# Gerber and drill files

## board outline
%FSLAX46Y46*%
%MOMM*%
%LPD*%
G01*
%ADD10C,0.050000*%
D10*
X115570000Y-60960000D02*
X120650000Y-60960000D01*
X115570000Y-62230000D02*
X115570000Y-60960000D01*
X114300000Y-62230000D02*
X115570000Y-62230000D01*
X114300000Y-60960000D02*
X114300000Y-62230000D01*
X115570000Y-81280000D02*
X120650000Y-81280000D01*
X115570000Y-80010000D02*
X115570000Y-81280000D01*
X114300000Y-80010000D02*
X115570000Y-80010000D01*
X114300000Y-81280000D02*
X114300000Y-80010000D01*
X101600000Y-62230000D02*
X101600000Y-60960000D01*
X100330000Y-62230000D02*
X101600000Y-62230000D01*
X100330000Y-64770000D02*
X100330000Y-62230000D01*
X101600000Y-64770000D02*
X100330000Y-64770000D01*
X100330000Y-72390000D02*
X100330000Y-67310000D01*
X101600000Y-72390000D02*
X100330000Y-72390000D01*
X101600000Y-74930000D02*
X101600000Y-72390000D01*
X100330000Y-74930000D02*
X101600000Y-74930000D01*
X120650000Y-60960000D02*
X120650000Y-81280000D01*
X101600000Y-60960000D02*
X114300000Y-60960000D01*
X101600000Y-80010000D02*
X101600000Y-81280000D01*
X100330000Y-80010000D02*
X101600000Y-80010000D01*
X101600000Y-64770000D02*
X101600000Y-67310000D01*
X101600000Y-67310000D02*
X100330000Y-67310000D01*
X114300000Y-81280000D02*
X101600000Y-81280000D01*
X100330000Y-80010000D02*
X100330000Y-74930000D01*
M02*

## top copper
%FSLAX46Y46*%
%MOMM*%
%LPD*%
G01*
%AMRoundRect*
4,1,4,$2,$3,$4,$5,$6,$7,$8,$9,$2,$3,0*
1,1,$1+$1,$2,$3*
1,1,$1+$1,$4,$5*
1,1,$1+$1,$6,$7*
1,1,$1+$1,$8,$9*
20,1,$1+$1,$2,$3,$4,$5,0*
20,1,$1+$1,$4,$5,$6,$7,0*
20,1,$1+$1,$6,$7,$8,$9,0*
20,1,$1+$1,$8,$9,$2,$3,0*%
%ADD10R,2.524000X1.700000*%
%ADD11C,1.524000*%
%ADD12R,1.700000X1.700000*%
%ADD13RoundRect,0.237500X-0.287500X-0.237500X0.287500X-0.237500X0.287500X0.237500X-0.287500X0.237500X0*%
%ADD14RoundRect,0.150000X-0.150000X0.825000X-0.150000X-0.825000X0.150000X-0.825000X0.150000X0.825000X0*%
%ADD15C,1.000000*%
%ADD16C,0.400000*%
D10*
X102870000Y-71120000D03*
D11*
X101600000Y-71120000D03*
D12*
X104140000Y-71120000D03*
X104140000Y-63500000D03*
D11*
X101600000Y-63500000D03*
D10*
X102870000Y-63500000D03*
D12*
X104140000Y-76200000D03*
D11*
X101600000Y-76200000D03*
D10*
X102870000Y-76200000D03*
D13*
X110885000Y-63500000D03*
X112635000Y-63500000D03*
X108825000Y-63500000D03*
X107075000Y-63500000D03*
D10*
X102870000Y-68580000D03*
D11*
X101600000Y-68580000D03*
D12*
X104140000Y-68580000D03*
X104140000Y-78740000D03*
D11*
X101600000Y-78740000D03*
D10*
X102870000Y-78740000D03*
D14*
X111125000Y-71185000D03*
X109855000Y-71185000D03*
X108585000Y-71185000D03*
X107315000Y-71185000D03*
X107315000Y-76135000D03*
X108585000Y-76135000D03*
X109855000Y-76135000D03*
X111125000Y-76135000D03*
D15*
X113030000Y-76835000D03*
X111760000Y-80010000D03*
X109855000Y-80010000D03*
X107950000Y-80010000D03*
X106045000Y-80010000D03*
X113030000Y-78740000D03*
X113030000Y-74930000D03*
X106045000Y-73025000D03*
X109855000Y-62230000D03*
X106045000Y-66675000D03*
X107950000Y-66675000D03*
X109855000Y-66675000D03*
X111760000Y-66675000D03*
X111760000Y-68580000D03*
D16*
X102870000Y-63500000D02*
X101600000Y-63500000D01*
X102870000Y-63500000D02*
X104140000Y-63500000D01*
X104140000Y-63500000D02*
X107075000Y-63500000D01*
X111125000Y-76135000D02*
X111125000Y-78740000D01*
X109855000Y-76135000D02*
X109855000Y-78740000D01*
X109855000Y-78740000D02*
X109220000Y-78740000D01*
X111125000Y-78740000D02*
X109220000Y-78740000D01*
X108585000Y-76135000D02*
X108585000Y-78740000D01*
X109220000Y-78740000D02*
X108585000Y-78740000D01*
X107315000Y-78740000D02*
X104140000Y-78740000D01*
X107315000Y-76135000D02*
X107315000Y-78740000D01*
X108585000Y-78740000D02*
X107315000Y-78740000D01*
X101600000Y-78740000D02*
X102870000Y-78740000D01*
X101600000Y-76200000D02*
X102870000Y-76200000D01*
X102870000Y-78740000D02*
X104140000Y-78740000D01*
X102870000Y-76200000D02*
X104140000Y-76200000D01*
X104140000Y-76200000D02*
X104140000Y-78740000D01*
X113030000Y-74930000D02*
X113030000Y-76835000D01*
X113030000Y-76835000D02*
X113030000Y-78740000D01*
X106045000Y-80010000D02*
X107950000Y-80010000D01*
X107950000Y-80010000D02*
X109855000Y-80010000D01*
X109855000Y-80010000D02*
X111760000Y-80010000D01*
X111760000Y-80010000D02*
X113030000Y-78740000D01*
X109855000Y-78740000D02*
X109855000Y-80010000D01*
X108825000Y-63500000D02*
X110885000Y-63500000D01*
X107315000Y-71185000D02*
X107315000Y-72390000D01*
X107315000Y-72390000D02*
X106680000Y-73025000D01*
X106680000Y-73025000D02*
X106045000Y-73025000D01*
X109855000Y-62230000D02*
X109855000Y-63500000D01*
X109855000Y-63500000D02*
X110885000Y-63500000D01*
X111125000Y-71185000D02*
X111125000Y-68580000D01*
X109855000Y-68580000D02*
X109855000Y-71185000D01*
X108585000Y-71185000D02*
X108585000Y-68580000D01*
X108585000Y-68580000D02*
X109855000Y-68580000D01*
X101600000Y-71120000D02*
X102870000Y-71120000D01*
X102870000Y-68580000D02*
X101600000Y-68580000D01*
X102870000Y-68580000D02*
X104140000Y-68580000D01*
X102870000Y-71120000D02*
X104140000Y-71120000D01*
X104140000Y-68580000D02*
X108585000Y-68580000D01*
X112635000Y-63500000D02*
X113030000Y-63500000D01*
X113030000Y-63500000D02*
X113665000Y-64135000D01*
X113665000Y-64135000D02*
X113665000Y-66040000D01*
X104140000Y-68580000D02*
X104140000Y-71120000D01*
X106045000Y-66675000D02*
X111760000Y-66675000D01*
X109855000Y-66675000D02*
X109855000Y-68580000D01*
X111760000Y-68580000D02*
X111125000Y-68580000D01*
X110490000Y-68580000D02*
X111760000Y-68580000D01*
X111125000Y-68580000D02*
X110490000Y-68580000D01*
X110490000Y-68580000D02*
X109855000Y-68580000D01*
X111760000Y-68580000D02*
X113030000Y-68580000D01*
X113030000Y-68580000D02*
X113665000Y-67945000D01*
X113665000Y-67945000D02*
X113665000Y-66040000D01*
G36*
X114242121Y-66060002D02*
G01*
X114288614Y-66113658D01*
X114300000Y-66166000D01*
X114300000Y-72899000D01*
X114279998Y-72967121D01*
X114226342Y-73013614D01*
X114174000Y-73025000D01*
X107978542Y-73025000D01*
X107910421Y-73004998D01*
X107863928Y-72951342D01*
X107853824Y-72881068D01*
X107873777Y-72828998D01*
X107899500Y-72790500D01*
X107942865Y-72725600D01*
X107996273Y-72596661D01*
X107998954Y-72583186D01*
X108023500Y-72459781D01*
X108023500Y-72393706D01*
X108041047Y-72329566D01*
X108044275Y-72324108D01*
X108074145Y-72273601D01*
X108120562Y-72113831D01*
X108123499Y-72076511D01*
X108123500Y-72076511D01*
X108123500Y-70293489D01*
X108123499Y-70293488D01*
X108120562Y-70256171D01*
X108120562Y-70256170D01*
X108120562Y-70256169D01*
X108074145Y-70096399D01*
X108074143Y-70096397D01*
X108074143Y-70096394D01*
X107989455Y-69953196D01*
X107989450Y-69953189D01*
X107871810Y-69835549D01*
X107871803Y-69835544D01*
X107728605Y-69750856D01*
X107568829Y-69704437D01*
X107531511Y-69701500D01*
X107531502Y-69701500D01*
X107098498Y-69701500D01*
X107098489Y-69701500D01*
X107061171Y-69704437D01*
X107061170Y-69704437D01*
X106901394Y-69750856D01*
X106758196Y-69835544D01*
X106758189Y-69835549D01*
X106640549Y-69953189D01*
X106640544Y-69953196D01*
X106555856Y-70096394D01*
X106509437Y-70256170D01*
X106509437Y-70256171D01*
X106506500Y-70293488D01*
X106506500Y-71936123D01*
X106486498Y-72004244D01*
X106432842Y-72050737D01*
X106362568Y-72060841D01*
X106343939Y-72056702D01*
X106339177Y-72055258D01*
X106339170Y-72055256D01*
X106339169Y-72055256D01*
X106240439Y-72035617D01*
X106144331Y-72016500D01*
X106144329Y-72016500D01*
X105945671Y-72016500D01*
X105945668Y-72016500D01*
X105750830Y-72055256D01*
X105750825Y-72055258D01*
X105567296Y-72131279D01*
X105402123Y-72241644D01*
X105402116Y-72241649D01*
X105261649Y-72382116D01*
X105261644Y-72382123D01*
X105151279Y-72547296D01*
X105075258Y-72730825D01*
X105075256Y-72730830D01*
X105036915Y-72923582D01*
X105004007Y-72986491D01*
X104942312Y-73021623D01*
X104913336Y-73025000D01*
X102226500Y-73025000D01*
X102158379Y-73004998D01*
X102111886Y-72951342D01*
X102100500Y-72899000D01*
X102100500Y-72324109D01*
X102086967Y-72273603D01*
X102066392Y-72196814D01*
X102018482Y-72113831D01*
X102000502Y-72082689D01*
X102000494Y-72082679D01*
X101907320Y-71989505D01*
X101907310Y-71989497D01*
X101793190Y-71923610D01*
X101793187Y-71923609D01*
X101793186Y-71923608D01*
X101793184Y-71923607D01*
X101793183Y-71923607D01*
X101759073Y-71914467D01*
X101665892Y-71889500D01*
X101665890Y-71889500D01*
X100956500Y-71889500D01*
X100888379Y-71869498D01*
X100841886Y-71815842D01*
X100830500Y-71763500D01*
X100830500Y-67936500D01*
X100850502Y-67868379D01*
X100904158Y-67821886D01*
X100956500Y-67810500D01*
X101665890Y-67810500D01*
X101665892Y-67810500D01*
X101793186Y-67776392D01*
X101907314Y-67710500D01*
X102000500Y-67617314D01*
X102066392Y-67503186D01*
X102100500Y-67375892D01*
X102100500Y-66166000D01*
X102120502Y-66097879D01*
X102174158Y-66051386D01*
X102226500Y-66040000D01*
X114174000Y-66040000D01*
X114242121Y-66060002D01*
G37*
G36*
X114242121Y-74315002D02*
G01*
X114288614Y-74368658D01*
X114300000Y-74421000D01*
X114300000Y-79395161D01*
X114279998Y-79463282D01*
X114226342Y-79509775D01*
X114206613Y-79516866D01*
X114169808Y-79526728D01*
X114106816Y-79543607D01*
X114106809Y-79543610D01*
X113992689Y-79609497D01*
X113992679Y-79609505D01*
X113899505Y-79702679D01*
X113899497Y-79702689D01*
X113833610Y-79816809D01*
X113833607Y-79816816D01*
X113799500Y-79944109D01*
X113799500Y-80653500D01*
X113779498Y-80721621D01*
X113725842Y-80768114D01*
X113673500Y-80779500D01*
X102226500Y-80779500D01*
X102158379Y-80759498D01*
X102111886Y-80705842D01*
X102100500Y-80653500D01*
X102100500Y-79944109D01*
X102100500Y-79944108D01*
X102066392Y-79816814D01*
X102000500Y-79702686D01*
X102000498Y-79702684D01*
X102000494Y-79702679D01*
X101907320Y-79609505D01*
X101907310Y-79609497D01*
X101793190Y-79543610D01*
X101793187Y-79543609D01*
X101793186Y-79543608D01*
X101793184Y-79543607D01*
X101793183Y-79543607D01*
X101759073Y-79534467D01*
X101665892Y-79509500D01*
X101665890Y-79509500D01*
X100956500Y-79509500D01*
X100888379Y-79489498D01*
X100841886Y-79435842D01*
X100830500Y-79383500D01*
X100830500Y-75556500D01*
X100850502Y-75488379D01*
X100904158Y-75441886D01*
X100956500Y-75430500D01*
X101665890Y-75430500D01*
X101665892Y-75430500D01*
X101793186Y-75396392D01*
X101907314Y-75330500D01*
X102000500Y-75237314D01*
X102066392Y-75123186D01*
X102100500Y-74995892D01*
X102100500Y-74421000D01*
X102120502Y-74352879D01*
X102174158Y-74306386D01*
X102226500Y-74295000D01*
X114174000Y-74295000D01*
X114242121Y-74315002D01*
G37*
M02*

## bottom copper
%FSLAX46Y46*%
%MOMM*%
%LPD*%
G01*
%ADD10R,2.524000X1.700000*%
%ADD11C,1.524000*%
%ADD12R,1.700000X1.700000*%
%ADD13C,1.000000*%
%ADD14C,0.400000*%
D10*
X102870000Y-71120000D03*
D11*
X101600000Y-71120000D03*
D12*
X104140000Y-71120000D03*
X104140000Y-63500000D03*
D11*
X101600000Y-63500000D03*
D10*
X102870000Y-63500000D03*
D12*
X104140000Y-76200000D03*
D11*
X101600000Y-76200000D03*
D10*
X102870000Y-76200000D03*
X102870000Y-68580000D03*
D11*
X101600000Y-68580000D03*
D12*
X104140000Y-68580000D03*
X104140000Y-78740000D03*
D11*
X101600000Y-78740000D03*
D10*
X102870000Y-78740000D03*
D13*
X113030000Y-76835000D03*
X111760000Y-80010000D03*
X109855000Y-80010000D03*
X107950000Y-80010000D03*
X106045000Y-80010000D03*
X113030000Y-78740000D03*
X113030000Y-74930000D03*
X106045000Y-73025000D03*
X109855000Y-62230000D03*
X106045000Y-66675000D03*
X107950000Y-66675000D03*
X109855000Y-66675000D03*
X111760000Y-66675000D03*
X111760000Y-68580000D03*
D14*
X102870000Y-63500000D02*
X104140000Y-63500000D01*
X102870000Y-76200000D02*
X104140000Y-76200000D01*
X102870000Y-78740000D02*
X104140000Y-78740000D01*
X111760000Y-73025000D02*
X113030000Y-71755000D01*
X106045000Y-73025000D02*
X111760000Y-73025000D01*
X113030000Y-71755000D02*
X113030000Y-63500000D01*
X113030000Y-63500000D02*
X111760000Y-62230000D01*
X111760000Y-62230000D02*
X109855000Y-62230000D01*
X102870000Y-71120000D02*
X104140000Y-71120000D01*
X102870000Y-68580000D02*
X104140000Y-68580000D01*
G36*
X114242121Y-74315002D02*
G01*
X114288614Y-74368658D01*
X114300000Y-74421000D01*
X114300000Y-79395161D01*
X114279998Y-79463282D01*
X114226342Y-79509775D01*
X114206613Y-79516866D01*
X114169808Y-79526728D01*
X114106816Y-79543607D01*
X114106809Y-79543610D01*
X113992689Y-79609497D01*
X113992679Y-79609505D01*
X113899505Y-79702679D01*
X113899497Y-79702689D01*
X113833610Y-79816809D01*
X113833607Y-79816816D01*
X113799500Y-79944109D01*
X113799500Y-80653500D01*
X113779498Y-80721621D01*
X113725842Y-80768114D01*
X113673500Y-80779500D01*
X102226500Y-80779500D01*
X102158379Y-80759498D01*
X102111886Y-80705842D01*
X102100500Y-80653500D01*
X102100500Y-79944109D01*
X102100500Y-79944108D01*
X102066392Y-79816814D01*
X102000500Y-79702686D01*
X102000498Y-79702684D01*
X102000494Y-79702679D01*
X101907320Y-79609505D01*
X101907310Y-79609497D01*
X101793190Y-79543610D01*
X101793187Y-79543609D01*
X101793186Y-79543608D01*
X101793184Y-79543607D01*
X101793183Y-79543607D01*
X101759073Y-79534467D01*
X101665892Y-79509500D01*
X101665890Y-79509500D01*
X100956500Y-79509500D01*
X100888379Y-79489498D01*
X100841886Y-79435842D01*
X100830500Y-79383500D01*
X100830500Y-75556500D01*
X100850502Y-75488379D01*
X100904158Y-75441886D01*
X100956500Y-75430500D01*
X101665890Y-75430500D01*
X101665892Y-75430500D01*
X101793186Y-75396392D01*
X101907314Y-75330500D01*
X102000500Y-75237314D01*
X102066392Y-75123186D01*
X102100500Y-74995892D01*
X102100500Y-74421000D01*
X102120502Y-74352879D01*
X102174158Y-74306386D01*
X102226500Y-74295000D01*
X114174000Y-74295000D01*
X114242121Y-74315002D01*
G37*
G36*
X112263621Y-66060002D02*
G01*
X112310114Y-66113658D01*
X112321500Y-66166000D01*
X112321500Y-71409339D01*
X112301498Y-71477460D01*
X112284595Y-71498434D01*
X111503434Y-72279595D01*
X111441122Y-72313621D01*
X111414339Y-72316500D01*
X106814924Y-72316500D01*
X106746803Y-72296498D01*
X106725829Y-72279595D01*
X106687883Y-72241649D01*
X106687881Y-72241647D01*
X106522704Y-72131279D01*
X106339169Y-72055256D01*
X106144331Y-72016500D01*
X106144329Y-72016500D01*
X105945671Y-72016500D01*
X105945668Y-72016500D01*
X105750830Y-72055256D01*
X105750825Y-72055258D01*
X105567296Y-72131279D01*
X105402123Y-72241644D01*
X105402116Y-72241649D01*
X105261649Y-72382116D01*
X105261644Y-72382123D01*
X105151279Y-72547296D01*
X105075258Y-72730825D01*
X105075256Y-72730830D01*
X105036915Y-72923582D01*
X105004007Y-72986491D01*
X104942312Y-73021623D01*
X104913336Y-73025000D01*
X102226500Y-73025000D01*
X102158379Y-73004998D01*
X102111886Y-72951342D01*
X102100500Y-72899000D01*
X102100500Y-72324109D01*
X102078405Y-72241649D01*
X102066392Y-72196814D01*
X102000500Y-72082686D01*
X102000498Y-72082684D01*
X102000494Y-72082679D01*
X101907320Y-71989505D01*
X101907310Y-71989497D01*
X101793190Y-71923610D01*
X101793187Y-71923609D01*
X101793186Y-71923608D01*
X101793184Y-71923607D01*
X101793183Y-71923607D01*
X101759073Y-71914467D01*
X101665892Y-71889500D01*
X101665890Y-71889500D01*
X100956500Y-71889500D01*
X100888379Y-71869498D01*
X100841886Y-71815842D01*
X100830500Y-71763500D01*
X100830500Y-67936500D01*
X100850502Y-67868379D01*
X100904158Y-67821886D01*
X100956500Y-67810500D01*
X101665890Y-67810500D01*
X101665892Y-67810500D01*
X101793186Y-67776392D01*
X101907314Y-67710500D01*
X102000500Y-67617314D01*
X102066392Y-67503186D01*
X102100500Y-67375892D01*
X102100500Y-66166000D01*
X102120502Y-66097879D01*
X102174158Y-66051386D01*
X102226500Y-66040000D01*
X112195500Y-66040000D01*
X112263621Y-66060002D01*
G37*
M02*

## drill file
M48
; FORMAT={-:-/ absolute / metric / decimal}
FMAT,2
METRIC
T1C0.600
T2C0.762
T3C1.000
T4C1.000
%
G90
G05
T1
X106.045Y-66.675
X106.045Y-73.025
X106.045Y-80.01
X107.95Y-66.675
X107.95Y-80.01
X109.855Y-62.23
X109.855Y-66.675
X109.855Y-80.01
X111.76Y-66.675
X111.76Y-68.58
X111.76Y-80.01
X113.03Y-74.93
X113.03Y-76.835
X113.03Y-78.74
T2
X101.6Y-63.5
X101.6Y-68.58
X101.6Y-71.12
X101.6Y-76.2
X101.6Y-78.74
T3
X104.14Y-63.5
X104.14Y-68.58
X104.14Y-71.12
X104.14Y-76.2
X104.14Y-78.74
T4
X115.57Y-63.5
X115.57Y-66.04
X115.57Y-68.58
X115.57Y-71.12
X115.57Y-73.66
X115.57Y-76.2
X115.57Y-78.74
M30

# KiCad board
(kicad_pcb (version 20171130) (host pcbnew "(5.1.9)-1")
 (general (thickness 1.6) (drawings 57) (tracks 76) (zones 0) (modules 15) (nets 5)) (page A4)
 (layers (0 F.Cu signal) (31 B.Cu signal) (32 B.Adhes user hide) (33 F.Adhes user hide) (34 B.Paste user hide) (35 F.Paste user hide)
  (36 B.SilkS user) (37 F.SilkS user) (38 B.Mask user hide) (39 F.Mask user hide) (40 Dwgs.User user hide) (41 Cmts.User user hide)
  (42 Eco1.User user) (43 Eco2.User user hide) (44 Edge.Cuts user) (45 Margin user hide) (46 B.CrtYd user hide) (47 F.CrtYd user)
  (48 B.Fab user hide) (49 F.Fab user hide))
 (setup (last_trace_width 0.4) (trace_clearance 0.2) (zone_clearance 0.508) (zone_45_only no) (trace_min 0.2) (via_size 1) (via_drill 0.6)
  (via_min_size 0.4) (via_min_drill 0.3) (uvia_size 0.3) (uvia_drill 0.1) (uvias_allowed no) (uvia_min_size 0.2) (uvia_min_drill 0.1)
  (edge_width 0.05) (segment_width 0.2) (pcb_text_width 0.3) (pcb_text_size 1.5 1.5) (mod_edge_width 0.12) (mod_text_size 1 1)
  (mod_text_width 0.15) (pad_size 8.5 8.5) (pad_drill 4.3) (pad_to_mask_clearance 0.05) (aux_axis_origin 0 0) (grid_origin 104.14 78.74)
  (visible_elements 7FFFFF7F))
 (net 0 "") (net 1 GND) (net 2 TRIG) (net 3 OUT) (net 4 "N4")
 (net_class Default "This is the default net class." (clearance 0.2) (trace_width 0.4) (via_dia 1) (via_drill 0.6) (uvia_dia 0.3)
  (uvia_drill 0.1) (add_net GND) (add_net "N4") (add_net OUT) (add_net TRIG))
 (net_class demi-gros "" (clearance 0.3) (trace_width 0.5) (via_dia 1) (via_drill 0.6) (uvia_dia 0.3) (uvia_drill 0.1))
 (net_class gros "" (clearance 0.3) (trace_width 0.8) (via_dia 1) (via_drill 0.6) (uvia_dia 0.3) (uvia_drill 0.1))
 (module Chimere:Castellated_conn (layer F.Cu) (at 104.14 71.12 180)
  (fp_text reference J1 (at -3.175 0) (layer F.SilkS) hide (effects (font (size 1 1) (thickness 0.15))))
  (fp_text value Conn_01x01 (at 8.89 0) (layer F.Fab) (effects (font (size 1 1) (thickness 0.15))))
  (pad 1 smd rect (at 1.27 0 180) (size 2.524 1.7) (layers B.Cu F.Paste F.Mask) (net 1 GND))
  (pad 1 smd rect (at 1.27 0 180) (size 2.524 1.7) (layers F.Cu F.Paste F.Mask) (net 1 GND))
  (pad 1 thru_hole circle (at 2.54 0 180) (size 1.524 1.524) (drill 0.762) (layers *.Cu *.Mask) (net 1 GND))
  (pad 1 thru_hole rect (at 0 0 180) (size 1.7 1.7) (drill 1) (layers *.Cu *.Mask) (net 1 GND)))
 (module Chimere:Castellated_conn (layer F.Cu) (at 104.14 63.5 180)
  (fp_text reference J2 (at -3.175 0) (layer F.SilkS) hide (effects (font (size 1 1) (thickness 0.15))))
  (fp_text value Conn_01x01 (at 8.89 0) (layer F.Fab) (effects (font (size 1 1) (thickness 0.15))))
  (pad 1 thru_hole rect (at 0 0 180) (size 1.7 1.7) (drill 1) (layers *.Cu *.Mask) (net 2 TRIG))
  (pad 1 thru_hole circle (at 2.54 0 180) (size 1.524 1.524) (drill 0.762) (layers *.Cu *.Mask) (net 2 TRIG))
  (pad 1 smd rect (at 1.27 0 180) (size 2.524 1.7) (layers F.Cu F.Paste F.Mask) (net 2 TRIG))
  (pad 1 smd rect (at 1.27 0 180) (size 2.524 1.7) (layers B.Cu F.Paste F.Mask) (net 2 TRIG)))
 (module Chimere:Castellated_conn (layer F.Cu) (at 104.14 76.2 180)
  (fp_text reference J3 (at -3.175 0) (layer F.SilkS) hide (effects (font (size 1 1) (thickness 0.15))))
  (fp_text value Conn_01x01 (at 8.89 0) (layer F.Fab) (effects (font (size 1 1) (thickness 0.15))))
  (pad 1 thru_hole rect (at 0 0 180) (size 1.7 1.7) (drill 1) (layers *.Cu *.Mask) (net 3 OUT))
  (pad 1 thru_hole circle (at 2.54 0 180) (size 1.524 1.524) (drill 0.762) (layers *.Cu *.Mask) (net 3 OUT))
  (pad 1 smd rect (at 1.27 0 180) (size 2.524 1.7) (layers F.Cu F.Paste F.Mask) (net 3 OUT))
  (pad 1 smd rect (at 1.27 0 180) (size 2.524 1.7) (layers B.Cu F.Paste F.Mask) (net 3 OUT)))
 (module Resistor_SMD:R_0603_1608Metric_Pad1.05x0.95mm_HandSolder (layer F.Cu) (at 111.76 63.5)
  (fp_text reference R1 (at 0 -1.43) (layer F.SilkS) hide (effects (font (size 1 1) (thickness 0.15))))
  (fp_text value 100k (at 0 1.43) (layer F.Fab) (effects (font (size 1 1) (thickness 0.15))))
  (pad 1 smd roundrect (at -0.875 0) (size 1.05 0.95) (layers F.Cu F.Paste F.Mask) (roundrect_rratio 0.25) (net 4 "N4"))
  (pad 2 smd roundrect (at 0.875 0) (size 1.05 0.95) (layers F.Cu F.Paste F.Mask) (roundrect_rratio 0.25) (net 1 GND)))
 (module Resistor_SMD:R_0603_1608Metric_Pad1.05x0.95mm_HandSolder (layer F.Cu) (at 107.95 63.5)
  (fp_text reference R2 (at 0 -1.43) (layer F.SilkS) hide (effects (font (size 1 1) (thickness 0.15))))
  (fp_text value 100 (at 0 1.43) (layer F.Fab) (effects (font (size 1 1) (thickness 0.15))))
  (pad 2 smd roundrect (at 0.875 0) (size 1.05 0.95) (layers F.Cu F.Paste F.Mask) (roundrect_rratio 0.25) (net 4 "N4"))
  (pad 1 smd roundrect (at -0.875 0) (size 1.05 0.95) (layers F.Cu F.Paste F.Mask) (roundrect_rratio 0.25) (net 2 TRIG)))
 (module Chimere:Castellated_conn (layer F.Cu) (at 104.14 68.58 180)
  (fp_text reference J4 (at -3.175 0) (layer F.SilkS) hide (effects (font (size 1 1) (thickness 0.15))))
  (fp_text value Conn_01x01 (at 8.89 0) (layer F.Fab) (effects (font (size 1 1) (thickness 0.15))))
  (pad 1 smd rect (at 1.27 0 180) (size 2.524 1.7) (layers B.Cu F.Paste F.Mask) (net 1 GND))
  (pad 1 smd rect (at 1.27 0 180) (size 2.524 1.7) (layers F.Cu F.Paste F.Mask) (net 1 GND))
  (pad 1 thru_hole circle (at 2.54 0 180) (size 1.524 1.524) (drill 0.762) (layers *.Cu *.Mask) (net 1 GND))
  (pad 1 thru_hole rect (at 0 0 180) (size 1.7 1.7) (drill 1) (layers *.Cu *.Mask) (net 1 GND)))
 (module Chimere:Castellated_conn (layer F.Cu) (at 104.14 78.74 180)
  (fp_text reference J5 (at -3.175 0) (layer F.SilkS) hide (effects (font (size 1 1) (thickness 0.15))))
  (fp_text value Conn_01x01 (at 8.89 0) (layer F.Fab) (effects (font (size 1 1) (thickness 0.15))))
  (pad 1 thru_hole rect (at 0 0 180) (size 1.7 1.7) (drill 1) (layers *.Cu *.Mask) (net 3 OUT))
  (pad 1 thru_hole circle (at 2.54 0 180) (size 1.524 1.524) (drill 0.762) (layers *.Cu *.Mask) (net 3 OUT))
  (pad 1 smd rect (at 1.27 0 180) (size 2.524 1.7) (layers F.Cu F.Paste F.Mask) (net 3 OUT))
  (pad 1 smd rect (at 1.27 0 180) (size 2.524 1.7) (layers B.Cu F.Paste F.Mask) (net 3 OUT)))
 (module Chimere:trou (layer F.Cu) (at 115.57 63.5)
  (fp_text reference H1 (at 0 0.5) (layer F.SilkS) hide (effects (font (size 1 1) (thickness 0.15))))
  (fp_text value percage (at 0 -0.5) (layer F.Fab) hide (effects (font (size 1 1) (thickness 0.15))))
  (pad "" np_thru_hole circle (at 0 0) (size 1 1) (drill 1) (layers *.Cu *.Mask)))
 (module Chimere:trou (layer F.Cu) (at 115.57 66.04)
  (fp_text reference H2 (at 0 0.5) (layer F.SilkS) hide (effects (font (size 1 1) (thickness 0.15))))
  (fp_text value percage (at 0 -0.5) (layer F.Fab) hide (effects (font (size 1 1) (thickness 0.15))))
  (pad "" np_thru_hole circle (at 0 0) (size 1 1) (drill 1) (layers *.Cu *.Mask)))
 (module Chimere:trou (layer F.Cu) (at 115.57 78.74)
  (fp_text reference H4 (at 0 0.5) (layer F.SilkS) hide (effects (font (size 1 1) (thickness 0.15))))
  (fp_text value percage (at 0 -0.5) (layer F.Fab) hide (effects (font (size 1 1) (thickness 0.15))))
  (pad "" np_thru_hole circle (at 0 0) (size 1 1) (drill 1) (layers *.Cu *.Mask)))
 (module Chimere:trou (layer F.Cu) (at 115.57 71.12)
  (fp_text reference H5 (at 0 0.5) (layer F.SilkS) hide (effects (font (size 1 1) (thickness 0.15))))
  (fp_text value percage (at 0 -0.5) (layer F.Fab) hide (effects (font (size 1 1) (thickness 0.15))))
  (pad "" np_thru_hole circle (at 0 0) (size 1 1) (drill 1) (layers *.Cu *.Mask)))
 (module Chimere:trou (layer F.Cu) (at 115.57 76.2)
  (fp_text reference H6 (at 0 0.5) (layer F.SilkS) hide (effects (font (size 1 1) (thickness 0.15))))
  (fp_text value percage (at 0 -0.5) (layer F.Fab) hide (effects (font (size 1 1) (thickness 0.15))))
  (pad "" np_thru_hole circle (at 0 0) (size 1 1) (drill 1) (layers *.Cu *.Mask)))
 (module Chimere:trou (layer F.Cu) (at 115.57 68.58)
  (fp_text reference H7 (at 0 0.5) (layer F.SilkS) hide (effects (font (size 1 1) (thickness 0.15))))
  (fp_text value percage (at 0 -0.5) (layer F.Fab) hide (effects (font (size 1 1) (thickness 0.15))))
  (pad "" np_thru_hole circle (at 0 0) (size 1 1) (drill 1) (layers *.Cu *.Mask)))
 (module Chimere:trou (layer F.Cu) (at 115.57 73.66)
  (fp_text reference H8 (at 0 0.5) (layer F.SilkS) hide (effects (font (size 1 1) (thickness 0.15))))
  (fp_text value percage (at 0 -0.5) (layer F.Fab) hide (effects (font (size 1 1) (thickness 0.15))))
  (pad "" np_thru_hole circle (at 0 0) (size 1 1) (drill 1) (layers *.Cu *.Mask)))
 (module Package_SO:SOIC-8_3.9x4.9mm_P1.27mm (layer F.Cu) (at 109.22 73.66 270)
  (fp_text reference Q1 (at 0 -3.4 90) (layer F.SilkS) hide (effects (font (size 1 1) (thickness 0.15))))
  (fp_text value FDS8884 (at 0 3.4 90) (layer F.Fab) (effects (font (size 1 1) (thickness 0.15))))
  (pad 1 smd roundrect (at -2.475 -1.905 270) (size 1.95 0.6) (layers F.Cu F.Paste F.Mask) (roundrect_rratio 0.25) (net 1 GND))
  (pad 2 smd roundrect (at -2.475 -0.635 270) (size 1.95 0.6) (layers F.Cu F.Paste F.Mask) (roundrect_rratio 0.25) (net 1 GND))
  (pad 3 smd roundrect (at -2.475 0.635 270) (size 1.95 0.6) (layers F.Cu F.Paste F.Mask) (roundrect_rratio 0.25) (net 1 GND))
  (pad 4 smd roundrect (at -2.475 1.905 270) (size 1.95 0.6) (layers F.Cu F.Paste F.Mask) (roundrect_rratio 0.25) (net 4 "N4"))
  (pad 5 smd roundrect (at 2.475 1.905 270) (size 1.95 0.6) (layers F.Cu F.Paste F.Mask) (roundrect_rratio 0.25) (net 3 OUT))
  (pad 6 smd roundrect (at 2.475 0.635 270) (size 1.95 0.6) (layers F.Cu F.Paste F.Mask) (roundrect_rratio 0.25) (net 3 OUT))
  (pad 7 smd roundrect (at 2.475 -0.635 270) (size 1.95 0.6) (layers F.Cu F.Paste F.Mask) (roundrect_rratio 0.25) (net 3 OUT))
  (pad 8 smd roundrect (at 2.475 -1.905 270) (size 1.95 0.6) (layers F.Cu F.Paste F.Mask) (roundrect_rratio 0.25) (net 3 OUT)))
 (gr_line (start 115.57 60.96) (end 120.65 60.96) (layer Edge.Cuts) (width 0.05))
 (gr_line (start 115.57 62.23) (end 115.57 60.96) (layer Edge.Cuts) (width 0.05))
 (gr_line (start 114.3 62.23) (end 115.57 62.23) (layer Edge.Cuts) (width 0.05))
 (gr_line (start 114.3 60.96) (end 114.3 62.23) (layer Edge.Cuts) (width 0.05))
 (gr_line (start 115.57 81.28) (end 120.65 81.28) (layer Edge.Cuts) (width 0.05))
 (gr_line (start 115.57 80.01) (end 115.57 81.28) (layer Edge.Cuts) (width 0.05))
 (gr_line (start 114.3 80.01) (end 115.57 80.01) (layer Edge.Cuts) (width 0.05))
 (gr_line (start 114.3 81.28) (end 114.3 80.01) (layer Edge.Cuts) (width 0.05))
 (gr_line (start 101.6 62.23) (end 101.6 60.96) (layer Edge.Cuts) (width 0.05))
 (gr_line (start 100.33 62.23) (end 101.6 62.23) (layer Edge.Cuts) (width 0.05))
 (gr_line (start 100.33 64.77) (end 100.33 62.23) (layer Edge.Cuts) (width 0.05))
 (gr_line (start 101.6 64.77) (end 100.33 64.77) (layer Edge.Cuts) (width 0.05))
 (gr_line (start 100.33 72.39) (end 100.33 67.31) (layer Edge.Cuts) (width 0.05))
 (gr_line (start 101.6 72.39) (end 100.33 72.39) (layer Edge.Cuts) (width 0.05))
 (gr_line (start 101.6 74.93) (end 101.6 72.39) (layer Edge.Cuts) (width 0.05))
 (gr_line (start 100.33 74.93) (end 101.6 74.93) (layer Edge.Cuts) (width 0.05))
 (gr_line (start 120.65 60.96) (end 120.65 81.28) (layer Edge.Cuts) (width 0.05))
 (gr_line (start 101.6 60.96) (end 114.3 60.96) (layer Edge.Cuts) (width 0.05))
 (gr_line (start 101.6 80.01) (end 101.6 81.28) (layer Edge.Cuts) (width 0.05))
 (gr_line (start 100.33 80.01) (end 101.6 80.01) (layer Edge.Cuts) (width 0.05))
 (gr_line (start 101.6 64.77) (end 101.6 67.31) (layer Edge.Cuts) (width 0.05))
 (gr_line (start 101.6 67.31) (end 100.33 67.31) (layer Edge.Cuts) (width 0.05))
 (gr_line (start 114.3 81.28) (end 101.6 81.28) (layer Edge.Cuts) (width 0.05))
 (gr_line (start 100.33 80.01) (end 100.33 74.93) (layer Edge.Cuts) (width 0.05))
 (segment (start 102.87 63.5) (end 104.14 63.5) (width 0.4) (layer B.Cu) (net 2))
 (segment (start 102.87 63.5) (end 101.6 63.5) (width 0.4) (layer F.Cu) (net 2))
 (segment (start 102.87 63.5) (end 104.14 63.5) (width 0.4) (layer F.Cu) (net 2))
 (segment (start 104.14 63.5) (end 107.075 63.5) (width 0.4) (layer F.Cu) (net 2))
 (via (at 113.03 76.835) (size 1) (drill 0.6) (layers F.Cu B.Cu) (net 3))
 (segment (start 111.125 76.135) (end 111.125 78.74) (width 0.4) (layer F.Cu) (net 3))
 (segment (start 109.855 76.135) (end 109.855 78.74) (width 0.4) (layer F.Cu) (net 3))
 (segment (start 109.855 78.74) (end 109.22 78.74) (width 0.4) (layer F.Cu) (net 3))
 (segment (start 111.125 78.74) (end 109.22 78.74) (width 0.4) (layer F.Cu) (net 3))
 (segment (start 108.585 76.135) (end 108.585 78.74) (width 0.4) (layer F.Cu) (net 3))
 (segment (start 109.22 78.74) (end 108.585 78.74) (width 0.4) (layer F.Cu) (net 3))
 (segment (start 107.315 78.74) (end 104.14 78.74) (width 0.4) (layer F.Cu) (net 3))
 (segment (start 107.315 76.135) (end 107.315 78.74) (width 0.4) (layer F.Cu) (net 3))
 (segment (start 108.585 78.74) (end 107.315 78.74) (width 0.4) (layer F.Cu) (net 3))
 (segment (start 101.6 78.74) (end 102.87 78.74) (width 0.4) (layer F.Cu) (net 3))
 (segment (start 101.6 76.2) (end 102.87 76.2) (width 0.4) (layer F.Cu) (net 3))
 (segment (start 102.87 78.74) (end 104.14 78.74) (width 0.4) (layer F.Cu) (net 3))
 (segment (start 102.87 76.2) (end 104.14 76.2) (width 0.4) (layer B.Cu) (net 3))
 (segment (start 102.87 78.74) (end 104.14 78.74) (width 0.4) (layer B.Cu) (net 3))
 (segment (start 102.87 76.2) (end 104.14 76.2) (width 0.4) (layer F.Cu) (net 3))
 (segment (start 104.14 76.2) (end 104.14 78.74) (width 0.4) (layer F.Cu) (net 3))
 (via (at 111.76 80.01) (size 1) (drill 0.6) (layers F.Cu B.Cu) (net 3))
 (via (at 109.855 80.01) (size 1) (drill 0.6) (layers F.Cu B.Cu) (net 3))
 (via (at 107.95 80.01) (size 1) (drill 0.6) (layers F.Cu B.Cu) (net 3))
 (via (at 106.045 80.01) (size 1) (drill 0.6) (layers F.Cu B.Cu) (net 3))
 (via (at 113.03 78.74) (size 1) (drill 0.6) (layers F.Cu B.Cu) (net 3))
 (via (at 113.03 74.93) (size 1) (drill 0.6) (layers F.Cu B.Cu) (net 3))
 (segment (start 113.03 74.93) (end 113.03 76.835) (width 0.4) (layer F.Cu) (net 3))
 (segment (start 113.03 76.835) (end 113.03 78.74) (width 0.4) (layer F.Cu) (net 3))
 (segment (start 106.045 80.01) (end 107.95 80.01) (width 0.4) (layer F.Cu) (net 3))
 (segment (start 107.95 80.01) (end 109.855 80.01) (width 0.4) (layer F.Cu) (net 3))
 (segment (start 109.855 80.01) (end 111.76 80.01) (width 0.4) (layer F.Cu) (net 3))
 (segment (start 111.76 80.01) (end 113.03 78.74) (width 0.4) (layer F.Cu) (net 3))
 (segment (start 109.855 78.74) (end 109.855 80.01) (width 0.4) (layer F.Cu) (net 3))
 (segment (start 108.825 63.5) (end 110.885 63.5) (width 0.4) (layer F.Cu) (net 4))
 (segment (start 107.315 71.185) (end 107.315 72.39) (width 0.4) (layer F.Cu) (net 4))
 (segment (start 107.315 72.39) (end 106.68 73.025) (width 0.4) (layer F.Cu) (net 4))
 (via (at 106.045 73.025) (size 1) (drill 0.6) (layers F.Cu B.Cu) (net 4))
 (segment (start 106.68 73.025) (end 106.045 73.025) (width 0.4) (layer F.Cu) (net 4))
 (via (at 109.855 62.23) (size 1) (drill 0.6) (layers F.Cu B.Cu) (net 4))
 (segment (start 109.855 62.23) (end 109.855 63.5) (width 0.4) (layer F.Cu) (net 4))
 (segment (start 109.855 63.5) (end 110.885 63.5) (width 0.4) (layer F.Cu) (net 4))
 (segment (start 111.76 73.025) (end 113.03 71.755) (width 0.4) (layer B.Cu) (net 4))
 (segment (start 106.045 73.025) (end 111.76 73.025) (width 0.4) (layer B.Cu) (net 4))
 (segment (start 113.03 71.755) (end 113.03 63.5) (width 0.4) (layer B.Cu) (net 4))
 (segment (start 113.03 63.5) (end 111.76 62.23) (width 0.4) (layer B.Cu) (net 4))
 (segment (start 111.76 62.23) (end 109.855 62.23) (width 0.4) (layer B.Cu) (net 4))
 (via (at 106.045 66.675) (size 1) (drill 0.6) (layers F.Cu B.Cu) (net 1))
 (segment (start 111.125 71.185) (end 111.125 68.58) (width 0.4) (layer F.Cu) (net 1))
 (segment (start 109.855 68.58) (end 109.855 71.185) (width 0.4) (layer F.Cu) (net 1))
 (segment (start 108.585 71.185) (end 108.585 68.58) (width 0.4) (layer F.Cu) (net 1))
 (segment (start 108.585 68.58) (end 109.855 68.58) (width 0.4) (layer F.Cu) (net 1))
 (segment (start 102.87 71.12) (end 104.14 71.12) (width 0.4) (layer B.Cu) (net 1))
 (segment (start 102.87 68.58) (end 104.14 68.58) (width 0.4) (layer B.Cu) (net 1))
 (segment (start 101.6 71.12) (end 102.87 71.12) (width 0.4) (layer F.Cu) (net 1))
 (segment (start 102.87 68.58) (end 101.6 68.58) (width 0.4) (layer F.Cu) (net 1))
 (segment (start 102.87 68.58) (end 104.14 68.58) (width 0.4) (layer F.Cu) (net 1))
 (segment (start 102.87 71.12) (end 104.14 71.12) (width 0.4) (layer F.Cu) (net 1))
 (segment (start 104.14 68.58) (end 108.585 68.58) (width 0.4) (layer F.Cu) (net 1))
 (segment (start 112.635 63.5) (end 113.03 63.5) (width 0.4) (layer F.Cu) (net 1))
 (segment (start 113.03 63.5) (end 113.665 64.135) (width 0.4) (layer F.Cu) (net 1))
 (segment (start 113.665 64.135) (end 113.665 66.04) (width 0.4) (layer F.Cu) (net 1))
 (segment (start 104.14 68.58) (end 104.14 71.12) (width 0.4) (layer F.Cu) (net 1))
 (via (at 107.95 66.675) (size 1) (drill 0.6) (layers F.Cu B.Cu) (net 1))
 (via (at 109.855 66.675) (size 1) (drill 0.6) (layers F.Cu B.Cu) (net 1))
 (via (at 111.76 66.675) (size 1) (drill 0.6) (layers F.Cu B.Cu) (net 1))
 (via (at 111.76 68.58) (size 1) (drill 0.6) (layers F.Cu B.Cu) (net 1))
 (segment (start 106.045 66.675) (end 111.76 66.675) (width 0.4) (layer F.Cu) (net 1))
 (segment (start 109.855 66.675) (end 109.855 68.58) (width 0.4) (layer F.Cu) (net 1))
 (segment (start 111.76 68.58) (end 111.125 68.58) (width 0.4) (layer F.Cu) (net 1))
 (segment (start 110.49 68.58) (end 111.76 68.58) (width 0.4) (layer F.Cu) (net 1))
 (segment (start 111.125 68.58) (end 110.49 68.58) (width 0.4) (layer F.Cu) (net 1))
 (segment (start 110.49 68.58) (end 109.855 68.58) (width 0.4) (layer F.Cu) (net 1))
 (segment (start 111.76 68.58) (end 113.03 68.58) (width 0.4) (layer F.Cu) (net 1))
 (segment (start 113.03 68.58) (end 113.665 67.945) (width 0.4) (layer F.Cu) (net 1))
 (segment (start 113.665 67.945) (end 113.665 66.04) (width 0.4) (layer F.Cu) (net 1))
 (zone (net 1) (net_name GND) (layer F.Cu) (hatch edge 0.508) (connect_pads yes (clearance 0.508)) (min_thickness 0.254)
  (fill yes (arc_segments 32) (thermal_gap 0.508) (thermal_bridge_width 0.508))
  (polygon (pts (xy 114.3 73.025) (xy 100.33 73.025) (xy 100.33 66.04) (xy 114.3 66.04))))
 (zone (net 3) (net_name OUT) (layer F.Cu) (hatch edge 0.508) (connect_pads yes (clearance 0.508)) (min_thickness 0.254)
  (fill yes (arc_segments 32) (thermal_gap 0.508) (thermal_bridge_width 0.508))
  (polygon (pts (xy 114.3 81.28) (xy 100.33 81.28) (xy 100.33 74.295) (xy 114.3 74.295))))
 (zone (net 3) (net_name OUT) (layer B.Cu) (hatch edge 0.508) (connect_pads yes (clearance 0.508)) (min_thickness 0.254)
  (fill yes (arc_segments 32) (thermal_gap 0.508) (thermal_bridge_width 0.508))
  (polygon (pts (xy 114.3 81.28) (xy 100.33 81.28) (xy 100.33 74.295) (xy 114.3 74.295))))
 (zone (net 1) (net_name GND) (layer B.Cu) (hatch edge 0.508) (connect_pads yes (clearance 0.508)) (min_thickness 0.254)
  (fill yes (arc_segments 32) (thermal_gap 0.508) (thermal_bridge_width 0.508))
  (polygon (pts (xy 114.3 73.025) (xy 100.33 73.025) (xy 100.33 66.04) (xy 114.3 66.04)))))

